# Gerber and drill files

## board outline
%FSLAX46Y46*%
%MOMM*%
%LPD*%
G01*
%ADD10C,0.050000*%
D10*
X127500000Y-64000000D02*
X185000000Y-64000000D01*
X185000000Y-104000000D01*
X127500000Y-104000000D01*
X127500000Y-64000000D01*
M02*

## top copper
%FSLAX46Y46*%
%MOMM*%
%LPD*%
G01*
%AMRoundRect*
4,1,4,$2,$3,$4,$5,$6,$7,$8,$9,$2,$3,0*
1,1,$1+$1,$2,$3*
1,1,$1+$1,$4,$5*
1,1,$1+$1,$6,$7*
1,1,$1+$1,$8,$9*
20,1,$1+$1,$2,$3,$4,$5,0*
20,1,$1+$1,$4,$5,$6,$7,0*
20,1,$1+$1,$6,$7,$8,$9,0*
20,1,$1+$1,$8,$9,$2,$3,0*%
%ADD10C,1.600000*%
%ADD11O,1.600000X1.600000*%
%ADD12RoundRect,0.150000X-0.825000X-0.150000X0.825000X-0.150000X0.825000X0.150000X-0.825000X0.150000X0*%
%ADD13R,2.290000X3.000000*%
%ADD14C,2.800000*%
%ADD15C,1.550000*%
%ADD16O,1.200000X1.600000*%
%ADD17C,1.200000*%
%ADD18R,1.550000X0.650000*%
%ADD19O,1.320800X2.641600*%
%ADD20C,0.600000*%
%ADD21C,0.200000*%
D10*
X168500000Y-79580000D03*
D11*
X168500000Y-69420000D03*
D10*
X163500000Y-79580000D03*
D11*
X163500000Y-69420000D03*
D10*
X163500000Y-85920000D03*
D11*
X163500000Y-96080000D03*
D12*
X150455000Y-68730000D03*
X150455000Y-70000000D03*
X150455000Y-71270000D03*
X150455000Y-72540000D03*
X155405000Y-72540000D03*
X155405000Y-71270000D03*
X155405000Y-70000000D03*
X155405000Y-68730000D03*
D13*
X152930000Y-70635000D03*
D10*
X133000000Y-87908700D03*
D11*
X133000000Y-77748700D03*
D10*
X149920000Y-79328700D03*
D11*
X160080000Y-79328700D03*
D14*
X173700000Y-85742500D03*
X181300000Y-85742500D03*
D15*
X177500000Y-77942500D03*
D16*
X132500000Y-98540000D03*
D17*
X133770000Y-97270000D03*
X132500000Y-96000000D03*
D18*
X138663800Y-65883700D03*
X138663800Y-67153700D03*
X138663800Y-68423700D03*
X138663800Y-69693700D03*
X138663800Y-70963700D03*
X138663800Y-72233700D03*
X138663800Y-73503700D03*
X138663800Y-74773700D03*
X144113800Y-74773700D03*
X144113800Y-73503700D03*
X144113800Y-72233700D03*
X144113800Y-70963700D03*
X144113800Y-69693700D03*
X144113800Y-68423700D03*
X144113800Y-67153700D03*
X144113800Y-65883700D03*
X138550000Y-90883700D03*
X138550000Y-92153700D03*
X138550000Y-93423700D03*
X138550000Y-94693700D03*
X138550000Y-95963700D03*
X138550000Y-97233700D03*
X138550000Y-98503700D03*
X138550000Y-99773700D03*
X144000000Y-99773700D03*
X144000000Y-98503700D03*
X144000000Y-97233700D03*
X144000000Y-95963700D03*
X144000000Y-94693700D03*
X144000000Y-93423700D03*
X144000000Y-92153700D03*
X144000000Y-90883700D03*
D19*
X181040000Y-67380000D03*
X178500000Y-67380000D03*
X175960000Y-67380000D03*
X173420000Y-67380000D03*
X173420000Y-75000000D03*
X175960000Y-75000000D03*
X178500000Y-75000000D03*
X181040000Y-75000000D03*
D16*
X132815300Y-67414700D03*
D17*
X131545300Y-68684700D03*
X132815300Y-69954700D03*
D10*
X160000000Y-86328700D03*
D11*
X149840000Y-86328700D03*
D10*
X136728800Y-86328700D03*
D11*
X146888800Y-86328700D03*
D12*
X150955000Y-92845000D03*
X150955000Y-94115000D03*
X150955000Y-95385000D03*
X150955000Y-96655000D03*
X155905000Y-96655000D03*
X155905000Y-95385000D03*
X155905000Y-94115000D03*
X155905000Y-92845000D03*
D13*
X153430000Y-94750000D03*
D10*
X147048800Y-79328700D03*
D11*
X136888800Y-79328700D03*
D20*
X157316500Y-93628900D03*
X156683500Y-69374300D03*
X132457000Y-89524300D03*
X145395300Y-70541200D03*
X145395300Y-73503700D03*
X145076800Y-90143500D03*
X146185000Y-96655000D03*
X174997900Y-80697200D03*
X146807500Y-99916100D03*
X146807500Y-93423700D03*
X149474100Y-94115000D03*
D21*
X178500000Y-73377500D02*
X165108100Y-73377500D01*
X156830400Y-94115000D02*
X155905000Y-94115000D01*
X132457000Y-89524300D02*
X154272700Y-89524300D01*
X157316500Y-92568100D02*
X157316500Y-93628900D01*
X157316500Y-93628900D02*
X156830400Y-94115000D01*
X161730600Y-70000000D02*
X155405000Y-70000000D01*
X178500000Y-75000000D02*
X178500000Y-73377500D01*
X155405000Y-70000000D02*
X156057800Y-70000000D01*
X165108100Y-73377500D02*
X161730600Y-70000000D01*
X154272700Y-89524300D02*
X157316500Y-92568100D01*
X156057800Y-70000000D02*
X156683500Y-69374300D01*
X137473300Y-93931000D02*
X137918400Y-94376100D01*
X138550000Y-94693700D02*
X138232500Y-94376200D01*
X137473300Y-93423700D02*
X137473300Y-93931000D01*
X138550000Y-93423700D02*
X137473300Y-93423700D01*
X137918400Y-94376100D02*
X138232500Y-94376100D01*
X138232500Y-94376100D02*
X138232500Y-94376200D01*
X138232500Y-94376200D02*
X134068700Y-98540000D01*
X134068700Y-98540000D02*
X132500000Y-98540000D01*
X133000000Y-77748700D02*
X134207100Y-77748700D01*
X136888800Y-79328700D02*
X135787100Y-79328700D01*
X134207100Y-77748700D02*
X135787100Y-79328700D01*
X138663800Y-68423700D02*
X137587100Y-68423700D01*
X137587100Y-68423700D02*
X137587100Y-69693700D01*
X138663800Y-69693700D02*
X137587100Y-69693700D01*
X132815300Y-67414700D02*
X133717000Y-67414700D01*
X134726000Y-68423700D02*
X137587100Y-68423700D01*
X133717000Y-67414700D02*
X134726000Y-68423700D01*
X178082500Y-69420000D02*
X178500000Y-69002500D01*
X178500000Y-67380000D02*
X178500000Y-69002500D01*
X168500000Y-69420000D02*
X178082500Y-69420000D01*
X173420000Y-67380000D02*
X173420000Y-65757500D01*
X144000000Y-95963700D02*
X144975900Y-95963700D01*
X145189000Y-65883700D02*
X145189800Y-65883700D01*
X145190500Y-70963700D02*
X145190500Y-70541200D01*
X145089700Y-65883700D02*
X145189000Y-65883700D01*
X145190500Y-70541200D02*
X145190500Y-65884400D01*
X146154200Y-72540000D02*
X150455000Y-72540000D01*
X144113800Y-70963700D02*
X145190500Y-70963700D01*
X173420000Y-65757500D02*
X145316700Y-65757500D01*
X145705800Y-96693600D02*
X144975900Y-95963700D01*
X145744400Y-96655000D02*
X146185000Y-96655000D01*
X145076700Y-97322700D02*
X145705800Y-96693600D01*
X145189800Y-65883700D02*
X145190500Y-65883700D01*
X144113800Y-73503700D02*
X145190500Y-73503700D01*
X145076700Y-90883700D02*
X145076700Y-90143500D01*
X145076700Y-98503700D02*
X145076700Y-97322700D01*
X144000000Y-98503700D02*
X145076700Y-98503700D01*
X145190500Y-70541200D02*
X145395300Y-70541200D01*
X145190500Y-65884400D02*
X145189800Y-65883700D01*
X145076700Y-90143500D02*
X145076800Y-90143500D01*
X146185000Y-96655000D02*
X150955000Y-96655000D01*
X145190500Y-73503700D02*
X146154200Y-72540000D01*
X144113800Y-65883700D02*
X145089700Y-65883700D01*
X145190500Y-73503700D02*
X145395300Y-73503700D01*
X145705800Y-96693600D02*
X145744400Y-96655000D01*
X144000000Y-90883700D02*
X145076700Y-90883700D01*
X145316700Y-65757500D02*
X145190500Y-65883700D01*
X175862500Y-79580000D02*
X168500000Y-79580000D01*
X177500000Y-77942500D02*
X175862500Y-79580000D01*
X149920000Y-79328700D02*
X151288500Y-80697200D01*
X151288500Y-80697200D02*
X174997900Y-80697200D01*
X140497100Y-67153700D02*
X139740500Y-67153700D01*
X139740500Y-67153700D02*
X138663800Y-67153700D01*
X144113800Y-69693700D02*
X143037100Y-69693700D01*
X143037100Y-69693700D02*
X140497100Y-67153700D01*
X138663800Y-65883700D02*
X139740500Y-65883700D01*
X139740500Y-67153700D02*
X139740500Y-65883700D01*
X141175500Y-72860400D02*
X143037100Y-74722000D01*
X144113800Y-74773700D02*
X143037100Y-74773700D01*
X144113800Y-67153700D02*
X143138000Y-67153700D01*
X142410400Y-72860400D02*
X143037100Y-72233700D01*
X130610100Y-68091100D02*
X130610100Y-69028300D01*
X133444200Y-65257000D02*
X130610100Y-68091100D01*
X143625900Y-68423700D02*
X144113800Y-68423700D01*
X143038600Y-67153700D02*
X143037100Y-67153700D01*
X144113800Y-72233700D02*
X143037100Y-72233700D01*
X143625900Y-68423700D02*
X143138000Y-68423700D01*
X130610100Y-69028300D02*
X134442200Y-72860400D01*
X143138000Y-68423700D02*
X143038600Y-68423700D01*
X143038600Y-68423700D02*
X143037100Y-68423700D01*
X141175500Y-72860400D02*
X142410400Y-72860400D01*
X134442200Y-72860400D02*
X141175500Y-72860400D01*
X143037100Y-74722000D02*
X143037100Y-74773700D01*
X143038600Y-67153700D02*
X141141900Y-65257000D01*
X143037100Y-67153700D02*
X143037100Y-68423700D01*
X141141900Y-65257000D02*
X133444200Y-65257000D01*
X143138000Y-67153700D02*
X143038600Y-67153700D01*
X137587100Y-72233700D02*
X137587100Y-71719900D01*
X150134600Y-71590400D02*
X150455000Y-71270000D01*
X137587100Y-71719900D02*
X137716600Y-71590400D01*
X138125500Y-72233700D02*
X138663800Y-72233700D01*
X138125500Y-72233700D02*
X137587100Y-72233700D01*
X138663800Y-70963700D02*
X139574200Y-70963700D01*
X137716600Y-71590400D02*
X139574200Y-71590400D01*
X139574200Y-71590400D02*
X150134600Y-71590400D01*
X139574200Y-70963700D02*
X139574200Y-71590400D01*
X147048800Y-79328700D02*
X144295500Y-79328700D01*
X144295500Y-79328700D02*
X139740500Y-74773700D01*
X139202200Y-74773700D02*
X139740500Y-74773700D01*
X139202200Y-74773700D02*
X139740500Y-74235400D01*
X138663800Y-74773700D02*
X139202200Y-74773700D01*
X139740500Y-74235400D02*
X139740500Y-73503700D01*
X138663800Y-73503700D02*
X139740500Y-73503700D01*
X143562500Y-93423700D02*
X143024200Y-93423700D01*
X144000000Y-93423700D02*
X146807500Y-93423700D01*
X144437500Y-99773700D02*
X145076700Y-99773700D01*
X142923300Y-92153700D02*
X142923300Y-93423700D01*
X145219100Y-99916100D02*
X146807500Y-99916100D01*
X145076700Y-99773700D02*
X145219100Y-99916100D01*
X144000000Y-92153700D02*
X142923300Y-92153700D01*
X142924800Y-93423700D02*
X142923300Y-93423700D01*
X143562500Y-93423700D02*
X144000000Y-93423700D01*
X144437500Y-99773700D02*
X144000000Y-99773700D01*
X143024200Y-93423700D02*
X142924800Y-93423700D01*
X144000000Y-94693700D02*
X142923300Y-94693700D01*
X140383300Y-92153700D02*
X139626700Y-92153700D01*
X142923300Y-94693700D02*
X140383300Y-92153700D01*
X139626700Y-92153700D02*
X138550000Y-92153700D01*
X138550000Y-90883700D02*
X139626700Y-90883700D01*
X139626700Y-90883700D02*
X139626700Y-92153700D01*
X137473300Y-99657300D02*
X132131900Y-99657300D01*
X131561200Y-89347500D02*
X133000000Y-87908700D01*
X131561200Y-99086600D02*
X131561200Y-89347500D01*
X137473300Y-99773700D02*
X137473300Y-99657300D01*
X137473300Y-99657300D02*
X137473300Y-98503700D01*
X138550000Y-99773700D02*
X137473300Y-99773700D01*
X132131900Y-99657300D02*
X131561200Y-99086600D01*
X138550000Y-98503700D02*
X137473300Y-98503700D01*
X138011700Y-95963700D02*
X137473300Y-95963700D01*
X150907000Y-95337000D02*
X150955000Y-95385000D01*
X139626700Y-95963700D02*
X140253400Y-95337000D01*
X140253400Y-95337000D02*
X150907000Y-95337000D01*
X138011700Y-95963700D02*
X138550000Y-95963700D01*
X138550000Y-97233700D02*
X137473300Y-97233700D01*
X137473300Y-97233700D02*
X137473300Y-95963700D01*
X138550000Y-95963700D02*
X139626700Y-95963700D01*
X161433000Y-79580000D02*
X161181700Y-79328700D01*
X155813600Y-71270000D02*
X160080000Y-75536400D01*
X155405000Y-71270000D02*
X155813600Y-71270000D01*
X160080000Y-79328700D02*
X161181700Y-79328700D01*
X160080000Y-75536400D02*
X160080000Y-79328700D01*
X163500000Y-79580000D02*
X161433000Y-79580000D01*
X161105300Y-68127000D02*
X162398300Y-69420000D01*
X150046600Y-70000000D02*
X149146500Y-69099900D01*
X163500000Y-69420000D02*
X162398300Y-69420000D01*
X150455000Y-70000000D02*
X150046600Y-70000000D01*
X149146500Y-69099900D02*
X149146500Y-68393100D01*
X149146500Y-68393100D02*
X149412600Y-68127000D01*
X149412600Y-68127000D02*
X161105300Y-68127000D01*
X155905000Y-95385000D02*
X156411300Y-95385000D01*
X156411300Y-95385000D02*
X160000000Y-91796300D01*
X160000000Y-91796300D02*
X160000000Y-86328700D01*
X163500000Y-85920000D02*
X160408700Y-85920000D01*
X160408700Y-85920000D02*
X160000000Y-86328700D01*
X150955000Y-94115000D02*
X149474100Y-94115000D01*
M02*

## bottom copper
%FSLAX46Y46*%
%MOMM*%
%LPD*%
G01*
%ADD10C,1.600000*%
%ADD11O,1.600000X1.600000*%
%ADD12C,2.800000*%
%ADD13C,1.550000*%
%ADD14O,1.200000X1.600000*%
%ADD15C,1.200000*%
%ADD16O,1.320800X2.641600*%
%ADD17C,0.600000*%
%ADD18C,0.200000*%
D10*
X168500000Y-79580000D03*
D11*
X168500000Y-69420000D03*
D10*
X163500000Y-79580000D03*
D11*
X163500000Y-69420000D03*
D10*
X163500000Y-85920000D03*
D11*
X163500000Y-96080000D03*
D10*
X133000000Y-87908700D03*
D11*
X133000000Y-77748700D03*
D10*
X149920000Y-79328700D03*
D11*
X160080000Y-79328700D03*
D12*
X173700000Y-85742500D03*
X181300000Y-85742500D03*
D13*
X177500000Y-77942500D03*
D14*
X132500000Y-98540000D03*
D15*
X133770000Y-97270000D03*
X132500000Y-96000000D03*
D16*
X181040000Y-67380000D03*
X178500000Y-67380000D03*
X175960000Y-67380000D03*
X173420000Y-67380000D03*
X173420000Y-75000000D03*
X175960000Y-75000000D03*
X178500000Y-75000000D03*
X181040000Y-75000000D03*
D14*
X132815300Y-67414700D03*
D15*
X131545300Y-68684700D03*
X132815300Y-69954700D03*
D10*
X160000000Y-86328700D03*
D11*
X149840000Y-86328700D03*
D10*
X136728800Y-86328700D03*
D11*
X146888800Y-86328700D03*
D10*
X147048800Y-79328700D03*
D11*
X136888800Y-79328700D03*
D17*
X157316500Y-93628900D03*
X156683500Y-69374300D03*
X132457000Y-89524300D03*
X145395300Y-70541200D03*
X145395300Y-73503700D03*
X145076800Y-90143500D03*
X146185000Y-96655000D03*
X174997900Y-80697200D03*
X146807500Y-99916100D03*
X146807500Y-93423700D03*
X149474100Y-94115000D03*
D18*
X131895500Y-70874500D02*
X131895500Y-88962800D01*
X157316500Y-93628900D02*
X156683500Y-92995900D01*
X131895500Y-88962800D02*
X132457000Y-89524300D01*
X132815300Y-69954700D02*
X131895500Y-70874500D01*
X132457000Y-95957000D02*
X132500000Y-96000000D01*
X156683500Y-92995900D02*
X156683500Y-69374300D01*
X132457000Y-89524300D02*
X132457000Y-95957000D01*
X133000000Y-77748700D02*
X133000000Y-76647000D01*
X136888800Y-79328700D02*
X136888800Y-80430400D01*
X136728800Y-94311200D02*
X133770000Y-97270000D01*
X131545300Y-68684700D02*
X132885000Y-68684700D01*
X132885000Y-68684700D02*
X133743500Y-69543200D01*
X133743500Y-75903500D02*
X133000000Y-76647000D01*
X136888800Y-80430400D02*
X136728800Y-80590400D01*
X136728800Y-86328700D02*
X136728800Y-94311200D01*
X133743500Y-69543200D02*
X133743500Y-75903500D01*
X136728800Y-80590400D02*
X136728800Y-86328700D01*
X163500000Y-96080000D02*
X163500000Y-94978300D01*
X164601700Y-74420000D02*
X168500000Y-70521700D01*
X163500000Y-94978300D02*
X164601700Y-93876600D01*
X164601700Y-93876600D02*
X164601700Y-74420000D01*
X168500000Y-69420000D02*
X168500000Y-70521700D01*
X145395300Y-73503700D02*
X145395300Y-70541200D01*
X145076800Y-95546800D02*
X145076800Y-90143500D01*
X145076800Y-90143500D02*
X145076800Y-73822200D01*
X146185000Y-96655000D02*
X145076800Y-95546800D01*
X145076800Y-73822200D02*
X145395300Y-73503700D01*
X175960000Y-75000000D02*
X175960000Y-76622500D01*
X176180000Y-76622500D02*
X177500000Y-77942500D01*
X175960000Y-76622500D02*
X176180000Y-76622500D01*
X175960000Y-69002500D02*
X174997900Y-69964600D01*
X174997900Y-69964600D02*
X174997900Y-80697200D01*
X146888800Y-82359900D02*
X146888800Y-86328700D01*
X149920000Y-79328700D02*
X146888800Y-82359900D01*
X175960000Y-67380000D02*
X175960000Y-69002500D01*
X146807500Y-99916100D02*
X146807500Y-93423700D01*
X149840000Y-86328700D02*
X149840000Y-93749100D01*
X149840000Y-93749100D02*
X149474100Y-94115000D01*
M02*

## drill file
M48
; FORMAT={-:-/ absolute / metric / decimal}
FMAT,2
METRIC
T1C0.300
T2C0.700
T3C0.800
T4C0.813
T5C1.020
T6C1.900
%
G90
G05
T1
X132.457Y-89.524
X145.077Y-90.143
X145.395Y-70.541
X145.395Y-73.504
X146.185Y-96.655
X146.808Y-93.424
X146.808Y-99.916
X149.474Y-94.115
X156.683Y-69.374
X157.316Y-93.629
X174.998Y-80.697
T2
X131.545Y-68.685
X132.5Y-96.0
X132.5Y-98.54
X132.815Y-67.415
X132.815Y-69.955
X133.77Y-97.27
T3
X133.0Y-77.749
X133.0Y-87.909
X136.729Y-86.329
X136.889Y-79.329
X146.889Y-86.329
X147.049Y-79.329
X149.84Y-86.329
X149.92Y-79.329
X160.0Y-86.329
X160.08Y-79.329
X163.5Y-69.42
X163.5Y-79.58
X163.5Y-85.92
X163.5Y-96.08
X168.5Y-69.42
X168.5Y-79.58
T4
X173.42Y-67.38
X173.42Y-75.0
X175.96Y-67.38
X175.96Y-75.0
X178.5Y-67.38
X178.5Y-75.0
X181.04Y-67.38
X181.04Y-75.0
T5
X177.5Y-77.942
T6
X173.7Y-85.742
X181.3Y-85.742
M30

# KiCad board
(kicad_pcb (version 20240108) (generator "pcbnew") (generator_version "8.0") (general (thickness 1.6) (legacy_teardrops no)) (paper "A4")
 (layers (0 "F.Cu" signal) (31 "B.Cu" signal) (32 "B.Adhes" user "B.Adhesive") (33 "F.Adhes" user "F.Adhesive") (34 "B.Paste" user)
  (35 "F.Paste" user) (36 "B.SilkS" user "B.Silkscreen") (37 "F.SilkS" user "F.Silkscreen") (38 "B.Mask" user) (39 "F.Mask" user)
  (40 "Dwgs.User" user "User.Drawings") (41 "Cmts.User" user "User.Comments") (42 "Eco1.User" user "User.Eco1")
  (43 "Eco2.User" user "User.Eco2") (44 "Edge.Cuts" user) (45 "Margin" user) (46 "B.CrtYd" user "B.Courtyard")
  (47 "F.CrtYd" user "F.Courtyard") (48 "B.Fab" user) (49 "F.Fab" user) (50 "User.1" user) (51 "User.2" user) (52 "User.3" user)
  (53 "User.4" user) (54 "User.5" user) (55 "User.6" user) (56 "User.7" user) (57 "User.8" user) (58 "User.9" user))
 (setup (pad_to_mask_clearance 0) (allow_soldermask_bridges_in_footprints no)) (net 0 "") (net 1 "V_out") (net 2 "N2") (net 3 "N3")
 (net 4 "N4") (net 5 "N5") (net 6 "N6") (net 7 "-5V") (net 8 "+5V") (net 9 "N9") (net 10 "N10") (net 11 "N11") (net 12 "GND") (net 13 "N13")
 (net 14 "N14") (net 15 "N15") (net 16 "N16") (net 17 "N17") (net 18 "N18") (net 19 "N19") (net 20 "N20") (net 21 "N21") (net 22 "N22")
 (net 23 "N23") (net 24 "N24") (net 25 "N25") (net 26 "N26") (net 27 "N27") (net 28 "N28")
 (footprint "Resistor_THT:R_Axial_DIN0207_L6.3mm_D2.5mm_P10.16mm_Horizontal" (layer "F.Cu") (at 168.5 79.58 90)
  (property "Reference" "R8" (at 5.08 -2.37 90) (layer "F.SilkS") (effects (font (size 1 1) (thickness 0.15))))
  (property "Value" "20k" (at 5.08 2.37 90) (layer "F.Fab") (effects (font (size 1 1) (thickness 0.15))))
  (pad "1" thru_hole circle (at 0 0 90) (size 1.6 1.6) (drill 0.8) (layers "*.Cu" "*.Mask") (remove_unused_layers no) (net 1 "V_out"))
  (pad "2" thru_hole oval (at 10.16 0 90) (size 1.6 1.6) (drill 0.8) (layers "*.Cu" "*.Mask") (remove_unused_layers no) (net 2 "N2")))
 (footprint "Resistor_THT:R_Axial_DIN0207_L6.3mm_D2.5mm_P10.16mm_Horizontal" (layer "F.Cu") (at 163.5 79.58 90)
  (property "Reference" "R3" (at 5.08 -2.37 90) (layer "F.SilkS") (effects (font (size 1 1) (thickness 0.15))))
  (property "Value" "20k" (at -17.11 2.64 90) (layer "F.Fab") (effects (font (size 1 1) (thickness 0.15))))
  (pad "1" thru_hole circle (at 0 0 90) (size 1.6 1.6) (drill 0.8) (layers "*.Cu" "*.Mask") (remove_unused_layers no) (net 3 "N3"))
  (pad "2" thru_hole oval (at 10.16 0 90) (size 1.6 1.6) (drill 0.8) (layers "*.Cu" "*.Mask") (remove_unused_layers no) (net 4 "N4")))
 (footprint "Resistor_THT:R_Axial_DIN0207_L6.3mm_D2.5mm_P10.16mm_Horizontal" (layer "F.Cu") (at 163.5 85.92 -90)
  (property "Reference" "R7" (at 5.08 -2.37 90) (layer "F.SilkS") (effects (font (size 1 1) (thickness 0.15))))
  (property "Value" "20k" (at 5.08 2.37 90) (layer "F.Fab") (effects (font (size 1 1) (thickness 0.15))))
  (pad "1" thru_hole circle (at 0 0 270) (size 1.6 1.6) (drill 0.8) (layers "*.Cu" "*.Mask") (remove_unused_layers no) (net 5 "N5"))
  (pad "2" thru_hole oval (at 10.16 0 270) (size 1.6 1.6) (drill 0.8) (layers "*.Cu" "*.Mask") (remove_unused_layers no) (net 2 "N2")))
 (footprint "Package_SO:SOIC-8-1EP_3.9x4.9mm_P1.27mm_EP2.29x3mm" (layer "F.Cu") (at 152.93 70.635)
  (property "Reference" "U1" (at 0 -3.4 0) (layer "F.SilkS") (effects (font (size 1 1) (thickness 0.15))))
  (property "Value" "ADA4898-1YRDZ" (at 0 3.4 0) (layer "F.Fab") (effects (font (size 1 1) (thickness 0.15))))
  (pad "" smd roundrect (at -0.57 -0.75) (size 0.92 1.21) (layers "F.Paste") (roundrect_rratio 0.25))
  (pad "" smd roundrect (at -0.57 0.75) (size 0.92 1.21) (layers "F.Paste") (roundrect_rratio 0.25))
  (pad "" smd roundrect (at 0.57 -0.75) (size 0.92 1.21) (layers "F.Paste") (roundrect_rratio 0.25))
  (pad "" smd roundrect (at 0.57 0.75) (size 0.92 1.21) (layers "F.Paste") (roundrect_rratio 0.25))
  (pad "1" smd roundrect (at -2.475 -1.905) (size 1.95 0.6) (layers "F.Cu" "F.Paste" "F.Mask") (roundrect_rratio 0.25))
  (pad "2" smd roundrect (at -2.475 -0.635) (size 1.95 0.6) (layers "F.Cu" "F.Paste" "F.Mask") (roundrect_rratio 0.25) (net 4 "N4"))
  (pad "3" smd roundrect (at -2.475 0.635) (size 1.95 0.6) (layers "F.Cu" "F.Paste" "F.Mask") (roundrect_rratio 0.25) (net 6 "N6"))
  (pad "4" smd roundrect (at -2.475 1.905) (size 1.95 0.6) (layers "F.Cu" "F.Paste" "F.Mask") (roundrect_rratio 0.25) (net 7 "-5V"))
  (pad "5" smd roundrect (at 2.475 1.905) (size 1.95 0.6) (layers "F.Cu" "F.Paste" "F.Mask") (roundrect_rratio 0.25))
  (pad "6" smd roundrect (at 2.475 0.635) (size 1.95 0.6) (layers "F.Cu" "F.Paste" "F.Mask") (roundrect_rratio 0.25) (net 3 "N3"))
  (pad "7" smd roundrect (at 2.475 -0.635) (size 1.95 0.6) (layers "F.Cu" "F.Paste" "F.Mask") (roundrect_rratio 0.25) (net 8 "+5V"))
  (pad "8" smd roundrect (at 2.475 -1.905) (size 1.95 0.6) (layers "F.Cu" "F.Paste" "F.Mask") (roundrect_rratio 0.25) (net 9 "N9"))
  (pad "9" smd rect (at 0 0) (size 2.29 3) (layers "F.Cu" "F.Mask") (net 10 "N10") (zone_connect 2)))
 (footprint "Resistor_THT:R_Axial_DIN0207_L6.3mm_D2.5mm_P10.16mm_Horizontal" (layer "F.Cu") (at 133 87.9087 90)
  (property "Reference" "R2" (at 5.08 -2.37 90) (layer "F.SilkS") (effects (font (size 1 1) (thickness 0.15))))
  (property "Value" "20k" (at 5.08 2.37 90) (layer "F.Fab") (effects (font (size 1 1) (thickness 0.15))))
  (pad "1" thru_hole circle (at 0 0 90) (size 1.6 1.6) (drill 0.8) (layers "*.Cu" "*.Mask") (remove_unused_layers no) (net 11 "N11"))
  (pad "2" thru_hole oval (at 10.16 0 90) (size 1.6 1.6) (drill 0.8) (layers "*.Cu" "*.Mask") (remove_unused_layers no) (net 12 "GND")))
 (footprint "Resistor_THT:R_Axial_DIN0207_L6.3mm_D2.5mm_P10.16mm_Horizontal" (layer "F.Cu") (at 149.92 79.3287)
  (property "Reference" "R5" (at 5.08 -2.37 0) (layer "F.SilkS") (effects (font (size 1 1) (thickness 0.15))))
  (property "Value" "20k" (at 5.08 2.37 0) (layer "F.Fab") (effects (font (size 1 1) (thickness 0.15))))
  (pad "1" thru_hole circle (at 0 0) (size 1.6 1.6) (drill 0.8) (layers "*.Cu" "*.Mask") (remove_unused_layers no) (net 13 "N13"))
  (pad "2" thru_hole oval (at 10.16 0) (size 1.6 1.6) (drill 0.8) (layers "*.Cu" "*.Mask") (remove_unused_layers no) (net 3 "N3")))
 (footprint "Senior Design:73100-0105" (layer "F.Cu") (at 177.5 103.3425)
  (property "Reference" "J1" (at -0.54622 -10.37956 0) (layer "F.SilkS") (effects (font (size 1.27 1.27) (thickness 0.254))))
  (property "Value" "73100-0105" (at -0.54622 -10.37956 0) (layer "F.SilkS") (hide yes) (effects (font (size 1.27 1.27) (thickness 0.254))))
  (pad "1" thru_hole circle (at -3.8 -17.6) (size 2.8 2.8) (drill 1.9) (layers "*.Cu" "*.Mask") (remove_unused_layers no) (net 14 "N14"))
  (pad "2" thru_hole circle (at 3.8 -17.6) (size 2.8 2.8) (drill 1.9) (layers "*.Cu" "*.Mask") (remove_unused_layers no) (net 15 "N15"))
  (pad "3" thru_hole circle (at 0 -25.4) (size 1.55 1.55) (drill 1.02) (layers "*.Cu" "*.Mask") (remove_unused_layers no) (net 1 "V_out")))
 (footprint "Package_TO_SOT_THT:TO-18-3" (layer "F.Cu") (at 132.5 98.54 90)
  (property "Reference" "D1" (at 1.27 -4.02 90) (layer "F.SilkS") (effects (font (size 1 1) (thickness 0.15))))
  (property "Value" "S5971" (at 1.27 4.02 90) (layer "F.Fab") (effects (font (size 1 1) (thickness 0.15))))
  (pad "1" thru_hole oval (at 0 0 90) (size 1.6 1.2) (drill 0.7) (layers "*.Cu" "*.Mask") (remove_unused_layers no) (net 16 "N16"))
  (pad "2" thru_hole circle (at 1.27 1.27 90) (size 1.2 1.2) (drill 0.7) (layers "*.Cu" "*.Mask") (remove_unused_layers no) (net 12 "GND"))
  (pad "3" thru_hole circle (at 2.54 0 90) (size 1.2 1.2) (drill 0.7) (layers "*.Cu" "*.Mask") (remove_unused_layers no) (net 8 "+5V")))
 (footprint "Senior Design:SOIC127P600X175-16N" (layer "F.Cu") (at 141.3888 70.3287)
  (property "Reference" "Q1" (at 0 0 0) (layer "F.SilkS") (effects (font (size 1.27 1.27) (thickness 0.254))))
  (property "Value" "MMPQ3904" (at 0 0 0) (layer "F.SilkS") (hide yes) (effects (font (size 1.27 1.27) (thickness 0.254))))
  (pad "1" smd rect (at -2.725 -4.445 90) (size 0.65 1.55) (layers "F.Cu" "F.Paste" "F.Mask") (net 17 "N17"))
  (pad "2" smd rect (at -2.725 -3.175 90) (size 0.65 1.55) (layers "F.Cu" "F.Paste" "F.Mask") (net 17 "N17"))
  (pad "3" smd rect (at -2.725 -1.905 90) (size 0.65 1.55) (layers "F.Cu" "F.Paste" "F.Mask") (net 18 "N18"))
  (pad "4" smd rect (at -2.725 -0.635 90) (size 0.65 1.55) (layers "F.Cu" "F.Paste" "F.Mask") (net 18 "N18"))
  (pad "5" smd rect (at -2.725 0.635 90) (size 0.65 1.55) (layers "F.Cu" "F.Paste" "F.Mask") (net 6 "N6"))
  (pad "6" smd rect (at -2.725 1.905 90) (size 0.65 1.55) (layers "F.Cu" "F.Paste" "F.Mask") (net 6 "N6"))
  (pad "7" smd rect (at -2.725 3.175 90) (size 0.65 1.55) (layers "F.Cu" "F.Paste" "F.Mask") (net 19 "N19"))
  (pad "8" smd rect (at -2.725 4.445 90) (size 0.65 1.55) (layers "F.Cu" "F.Paste" "F.Mask") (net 19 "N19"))
  (pad "9" smd rect (at 2.725 4.445 90) (size 0.65 1.55) (layers "F.Cu" "F.Paste" "F.Mask") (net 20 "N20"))
  (pad "10" smd rect (at 2.725 3.175 90) (size 0.65 1.55) (layers "F.Cu" "F.Paste" "F.Mask") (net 7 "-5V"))
  (pad "11" smd rect (at 2.725 1.905 90) (size 0.65 1.55) (layers "F.Cu" "F.Paste" "F.Mask") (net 20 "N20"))
  (pad "12" smd rect (at 2.725 0.635 90) (size 0.65 1.55) (layers "F.Cu" "F.Paste" "F.Mask") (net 7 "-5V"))
  (pad "13" smd rect (at 2.725 -0.635 90) (size 0.65 1.55) (layers "F.Cu" "F.Paste" "F.Mask") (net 17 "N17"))
  (pad "14" smd rect (at 2.725 -1.905 90) (size 0.65 1.55) (layers "F.Cu" "F.Paste" "F.Mask") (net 20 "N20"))
  (pad "15" smd rect (at 2.725 -3.175 90) (size 0.65 1.55) (layers "F.Cu" "F.Paste" "F.Mask") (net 20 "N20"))
  (pad "16" smd rect (at 2.725 -4.445 90) (size 0.65 1.55) (layers "F.Cu" "F.Paste" "F.Mask") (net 7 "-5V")))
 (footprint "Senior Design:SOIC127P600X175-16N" (layer "F.Cu") (at 141.275 95.3287)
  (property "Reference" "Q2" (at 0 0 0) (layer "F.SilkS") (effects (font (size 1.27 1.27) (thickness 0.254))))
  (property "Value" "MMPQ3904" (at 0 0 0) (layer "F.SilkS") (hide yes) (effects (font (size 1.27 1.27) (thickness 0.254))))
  (pad "1" smd rect (at -2.725 -4.445 90) (size 0.65 1.55) (layers "F.Cu" "F.Paste" "F.Mask") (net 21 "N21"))
  (pad "2" smd rect (at -2.725 -3.175 90) (size 0.65 1.55) (layers "F.Cu" "F.Paste" "F.Mask") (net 21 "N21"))
  (pad "3" smd rect (at -2.725 -1.905 90) (size 0.65 1.55) (layers "F.Cu" "F.Paste" "F.Mask") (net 16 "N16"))
  (pad "4" smd rect (at -2.725 -0.635 90) (size 0.65 1.55) (layers "F.Cu" "F.Paste" "F.Mask") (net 16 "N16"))
  (pad "5" smd rect (at -2.725 0.635 90) (size 0.65 1.55) (layers "F.Cu" "F.Paste" "F.Mask") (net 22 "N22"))
  (pad "6" smd rect (at -2.725 1.905 90) (size 0.65 1.55) (layers "F.Cu" "F.Paste" "F.Mask") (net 22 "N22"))
  (pad "7" smd rect (at -2.725 3.175 90) (size 0.65 1.55) (layers "F.Cu" "F.Paste" "F.Mask") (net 11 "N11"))
  (pad "8" smd rect (at -2.725 4.445 90) (size 0.65 1.55) (layers "F.Cu" "F.Paste" "F.Mask") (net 11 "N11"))
  (pad "9" smd rect (at 2.725 4.445 90) (size 0.65 1.55) (layers "F.Cu" "F.Paste" "F.Mask") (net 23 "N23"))
  (pad "10" smd rect (at 2.725 3.175 90) (size 0.65 1.55) (layers "F.Cu" "F.Paste" "F.Mask") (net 7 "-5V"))
  (pad "11" smd rect (at 2.725 1.905 90) (size 0.65 1.55) (layers "F.Cu" "F.Paste" "F.Mask") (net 23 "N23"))
  (pad "12" smd rect (at 2.725 0.635 90) (size 0.65 1.55) (layers "F.Cu" "F.Paste" "F.Mask") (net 7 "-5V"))
  (pad "13" smd rect (at 2.725 -0.635 90) (size 0.65 1.55) (layers "F.Cu" "F.Paste" "F.Mask") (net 21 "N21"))
  (pad "14" smd rect (at 2.725 -1.905 90) (size 0.65 1.55) (layers "F.Cu" "F.Paste" "F.Mask") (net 23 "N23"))
  (pad "15" smd rect (at 2.725 -3.175 90) (size 0.65 1.55) (layers "F.Cu" "F.Paste" "F.Mask") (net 23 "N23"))
  (pad "16" smd rect (at 2.725 -4.445 90) (size 0.65 1.55) (layers "F.Cu" "F.Paste" "F.Mask") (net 7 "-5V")))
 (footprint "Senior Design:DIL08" (layer "F.Cu") (at 177.23 71.19 180)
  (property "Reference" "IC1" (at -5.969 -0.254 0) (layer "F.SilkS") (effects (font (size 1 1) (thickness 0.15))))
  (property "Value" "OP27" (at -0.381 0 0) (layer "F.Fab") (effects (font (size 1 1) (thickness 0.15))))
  (pad "1" thru_hole oval (at -3.81 3.81 180) (size 1.3208 2.6416) (drill 0.8128) (layers "*.Cu" "*.Mask") (remove_unused_layers no)
   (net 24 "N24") (solder_mask_margin 0.102))
  (pad "2" thru_hole oval (at -1.27 3.81 180) (size 1.3208 2.6416) (drill 0.8128) (layers "*.Cu" "*.Mask") (remove_unused_layers no)
   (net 2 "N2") (solder_mask_margin 0.102))
  (pad "3" thru_hole oval (at 1.27 3.81 180) (size 1.3208 2.6416) (drill 0.8128) (layers "*.Cu" "*.Mask") (remove_unused_layers no)
   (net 13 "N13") (solder_mask_margin 0.102))
  (pad "4" thru_hole oval (at 3.81 3.81 180) (size 1.3208 2.6416) (drill 0.8128) (layers "*.Cu" "*.Mask") (remove_unused_layers no)
   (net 7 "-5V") (solder_mask_margin 0.102))
  (pad "5" thru_hole oval (at 3.81 -3.81 180) (size 1.3208 2.6416) (drill 0.8128) (layers "*.Cu" "*.Mask") (remove_unused_layers no)
   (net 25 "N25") (solder_mask_margin 0.102))
  (pad "6" thru_hole oval (at 1.27 -3.81 180) (size 1.3208 2.6416) (drill 0.8128) (layers "*.Cu" "*.Mask") (remove_unused_layers no)
   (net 1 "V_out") (solder_mask_margin 0.102))
  (pad "7" thru_hole oval (at -1.27 -3.81 180) (size 1.3208 2.6416) (drill 0.8128) (layers "*.Cu" "*.Mask") (remove_unused_layers no)
   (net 8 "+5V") (solder_mask_margin 0.102))
  (pad "8" thru_hole oval (at -3.81 -3.81 180) (size 1.3208 2.6416) (drill 0.8128) (layers "*.Cu" "*.Mask") (remove_unused_layers no)
   (solder_mask_margin 0.102)))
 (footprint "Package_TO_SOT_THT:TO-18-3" (layer "F.Cu") (at 132.8153 67.4147 -90)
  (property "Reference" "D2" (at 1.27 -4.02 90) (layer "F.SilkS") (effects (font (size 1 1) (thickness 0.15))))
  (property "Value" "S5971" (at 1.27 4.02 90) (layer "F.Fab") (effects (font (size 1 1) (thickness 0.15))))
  (pad "1" thru_hole oval (at 0 0 270) (size 1.6 1.2) (drill 0.7) (layers "*.Cu" "*.Mask") (remove_unused_layers no) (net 18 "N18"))
  (pad "2" thru_hole circle (at 1.27 1.27 270) (size 1.2 1.2) (drill 0.7) (layers "*.Cu" "*.Mask") (remove_unused_layers no) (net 12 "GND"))
  (pad "3" thru_hole circle (at 2.54 0 270) (size 1.2 1.2) (drill 0.7) (layers "*.Cu" "*.Mask") (remove_unused_layers no) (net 8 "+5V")))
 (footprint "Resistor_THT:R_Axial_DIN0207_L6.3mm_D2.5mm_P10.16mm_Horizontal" (layer "F.Cu") (at 160 86.3287 180)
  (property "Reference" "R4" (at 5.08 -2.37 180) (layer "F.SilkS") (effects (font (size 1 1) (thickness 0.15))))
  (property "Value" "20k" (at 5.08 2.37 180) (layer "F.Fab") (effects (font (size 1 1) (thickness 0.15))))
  (pad "1" thru_hole circle (at 0 0 180) (size 1.6 1.6) (drill 0.8) (layers "*.Cu" "*.Mask") (remove_unused_layers no) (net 5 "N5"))
  (pad "2" thru_hole oval (at 10.16 0 180) (size 1.6 1.6) (drill 0.8) (layers "*.Cu" "*.Mask") (remove_unused_layers no) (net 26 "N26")))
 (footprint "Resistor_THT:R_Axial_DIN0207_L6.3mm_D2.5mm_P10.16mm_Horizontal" (layer "F.Cu") (at 136.7288 86.3287)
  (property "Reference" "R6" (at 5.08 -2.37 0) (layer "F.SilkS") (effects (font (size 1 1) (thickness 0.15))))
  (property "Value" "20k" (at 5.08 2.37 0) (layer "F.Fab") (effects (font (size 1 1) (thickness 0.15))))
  (pad "1" thru_hole circle (at 0 0) (size 1.6 1.6) (drill 0.8) (layers "*.Cu" "*.Mask") (remove_unused_layers no) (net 12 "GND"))
  (pad "2" thru_hole oval (at 10.16 0) (size 1.6 1.6) (drill 0.8) (layers "*.Cu" "*.Mask") (remove_unused_layers no) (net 13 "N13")))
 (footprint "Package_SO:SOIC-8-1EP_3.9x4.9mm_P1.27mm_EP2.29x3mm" (layer "F.Cu") (at 153.43 94.75)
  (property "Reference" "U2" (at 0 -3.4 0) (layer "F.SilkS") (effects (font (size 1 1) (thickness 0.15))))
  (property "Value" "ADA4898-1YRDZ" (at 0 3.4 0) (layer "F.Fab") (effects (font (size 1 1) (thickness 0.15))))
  (pad "" smd roundrect (at -0.57 -0.75) (size 0.92 1.21) (layers "F.Paste") (roundrect_rratio 0.25))
  (pad "" smd roundrect (at -0.57 0.75) (size 0.92 1.21) (layers "F.Paste") (roundrect_rratio 0.25))
  (pad "" smd roundrect (at 0.57 -0.75) (size 0.92 1.21) (layers "F.Paste") (roundrect_rratio 0.25))
  (pad "" smd roundrect (at 0.57 0.75) (size 0.92 1.21) (layers "F.Paste") (roundrect_rratio 0.25))
  (pad "1" smd roundrect (at -2.475 -1.905) (size 1.95 0.6) (layers "F.Cu" "F.Paste" "F.Mask") (roundrect_rratio 0.25))
  (pad "2" smd roundrect (at -2.475 -0.635) (size 1.95 0.6) (layers "F.Cu" "F.Paste" "F.Mask") (roundrect_rratio 0.25) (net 26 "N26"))
  (pad "3" smd roundrect (at -2.475 0.635) (size 1.95 0.6) (layers "F.Cu" "F.Paste" "F.Mask") (roundrect_rratio 0.25) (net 22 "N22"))
  (pad "4" smd roundrect (at -2.475 1.905) (size 1.95 0.6) (layers "F.Cu" "F.Paste" "F.Mask") (roundrect_rratio 0.25) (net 7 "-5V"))
  (pad "5" smd roundrect (at 2.475 1.905) (size 1.95 0.6) (layers "F.Cu" "F.Paste" "F.Mask") (roundrect_rratio 0.25))
  (pad "6" smd roundrect (at 2.475 0.635) (size 1.95 0.6) (layers "F.Cu" "F.Paste" "F.Mask") (roundrect_rratio 0.25) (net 5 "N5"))
  (pad "7" smd roundrect (at 2.475 -0.635) (size 1.95 0.6) (layers "F.Cu" "F.Paste" "F.Mask") (roundrect_rratio 0.25) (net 8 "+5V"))
  (pad "8" smd roundrect (at 2.475 -1.905) (size 1.95 0.6) (layers "F.Cu" "F.Paste" "F.Mask") (roundrect_rratio 0.25) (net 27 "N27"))
  (pad "9" smd rect (at 0 0) (size 2.29 3) (layers "F.Cu" "F.Mask") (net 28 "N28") (zone_connect 2)))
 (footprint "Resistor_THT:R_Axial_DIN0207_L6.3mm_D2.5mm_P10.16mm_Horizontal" (layer "F.Cu") (at 147.0488 79.3287 180)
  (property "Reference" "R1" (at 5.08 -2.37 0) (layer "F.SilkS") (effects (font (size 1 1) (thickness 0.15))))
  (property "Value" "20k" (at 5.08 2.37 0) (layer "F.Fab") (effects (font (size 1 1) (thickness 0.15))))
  (pad "1" thru_hole circle (at 0 0 180) (size 1.6 1.6) (drill 0.8) (layers "*.Cu" "*.Mask") (remove_unused_layers no) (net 19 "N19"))
  (pad "2" thru_hole oval (at 10.16 0 180) (size 1.6 1.6) (drill 0.8) (layers "*.Cu" "*.Mask") (remove_unused_layers no) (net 12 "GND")))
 (gr_rect (start 127.5 64) (end 185 104) (stroke (width 0.05) (type default)) (fill none) (layer "Edge.Cuts"))
 (segment (start 178.5 73.3775) (end 165.1081 73.3775) (width 0.2) (layer "F.Cu") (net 8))
 (segment (start 156.8304 94.115) (end 155.905 94.115) (width 0.2) (layer "F.Cu") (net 8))
 (segment (start 132.457 89.5243) (end 154.2727 89.5243) (width 0.2) (layer "F.Cu") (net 8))
 (segment (start 157.3165 92.5681) (end 157.3165 93.6289) (width 0.2) (layer "F.Cu") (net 8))
 (segment (start 157.3165 93.6289) (end 156.8304 94.115) (width 0.2) (layer "F.Cu") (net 8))
 (segment (start 161.7306 70) (end 155.405 70) (width 0.2) (layer "F.Cu") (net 8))
 (segment (start 178.5 75) (end 178.5 73.3775) (width 0.2) (layer "F.Cu") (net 8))
 (segment (start 155.405 70) (end 156.0578 70) (width 0.2) (layer "F.Cu") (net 8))
 (segment (start 165.1081 73.3775) (end 161.7306 70) (width 0.2) (layer "F.Cu") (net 8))
 (segment (start 154.2727 89.5243) (end 157.3165 92.5681) (width 0.2) (layer "F.Cu") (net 8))
 (segment (start 156.0578 70) (end 156.6835 69.3743) (width 0.2) (layer "F.Cu") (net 8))
 (via (at 157.3165 93.6289) (size 0.6) (drill 0.3) (layers "F.Cu" "B.Cu") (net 8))
 (via (at 156.6835 69.3743) (size 0.6) (drill 0.3) (layers "F.Cu" "B.Cu") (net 8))
 (via (at 132.457 89.5243) (size 0.6) (drill 0.3) (layers "F.Cu" "B.Cu") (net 8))
 (segment (start 131.8955 70.8745) (end 131.8955 88.9628) (width 0.2) (layer "B.Cu") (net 8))
 (segment (start 157.3165 93.6289) (end 156.6835 92.9959) (width 0.2) (layer "B.Cu") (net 8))
 (segment (start 131.8955 88.9628) (end 132.457 89.5243) (width 0.2) (layer "B.Cu") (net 8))
 (segment (start 132.8153 69.9547) (end 131.8955 70.8745) (width 0.2) (layer "B.Cu") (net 8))
 (segment (start 132.457 95.957) (end 132.5 96) (width 0.2) (layer "B.Cu") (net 8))
 (segment (start 156.6835 92.9959) (end 156.6835 69.3743) (width 0.2) (layer "B.Cu") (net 8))
 (segment (start 132.457 89.5243) (end 132.457 95.957) (width 0.2) (layer "B.Cu") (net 8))
 (segment (start 137.4733 93.931) (end 137.9184 94.3761) (width 0.2) (layer "F.Cu") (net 16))
 (segment (start 138.55 94.6937) (end 138.2325 94.3762) (width 0.2) (layer "F.Cu") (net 16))
 (segment (start 137.4733 93.4237) (end 137.4733 93.931) (width 0.2) (layer "F.Cu") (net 16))
 (segment (start 138.55 93.4237) (end 137.4733 93.4237) (width 0.2) (layer "F.Cu") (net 16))
 (segment (start 137.9184 94.3761) (end 138.2325 94.3761) (width 0.2) (layer "F.Cu") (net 16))
 (segment (start 138.2325 94.3761) (end 138.2325 94.3762) (width 0.2) (layer "F.Cu") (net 16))
 (segment (start 138.2325 94.3762) (end 134.0687 98.54) (width 0.2) (layer "F.Cu") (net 16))
 (segment (start 134.0687 98.54) (end 132.5 98.54) (width 0.2) (layer "F.Cu") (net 16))
 (segment (start 133 77.7487) (end 134.2071 77.7487) (width 0.2) (layer "F.Cu") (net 12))
 (segment (start 136.8888 79.3287) (end 135.7871 79.3287) (width 0.2) (layer "F.Cu") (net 12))
 (segment (start 134.2071 77.7487) (end 135.7871 79.3287) (width 0.2) (layer "F.Cu") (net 12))
 (segment (start 133 77.7487) (end 133 76.647) (width 0.2) (layer "B.Cu") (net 12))
 (segment (start 136.8888 79.3287) (end 136.8888 80.4304) (width 0.2) (layer "B.Cu") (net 12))
 (segment (start 136.7288 94.3112) (end 133.77 97.27) (width 0.2) (layer "B.Cu") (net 12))
 (segment (start 131.5453 68.6847) (end 132.885 68.6847) (width 0.2) (layer "B.Cu") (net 12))
 (segment (start 132.885 68.6847) (end 133.7435 69.5432) (width 0.2) (layer "B.Cu") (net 12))
 (segment (start 133.7435 75.9035) (end 133 76.647) (width 0.2) (layer "B.Cu") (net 12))
 (segment (start 136.8888 80.4304) (end 136.7288 80.5904) (width 0.2) (layer "B.Cu") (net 12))
 (segment (start 136.7288 86.3287) (end 136.7288 94.3112) (width 0.2) (layer "B.Cu") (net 12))
 (segment (start 133.7435 69.5432) (end 133.7435 75.9035) (width 0.2) (layer "B.Cu") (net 12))
 (segment (start 136.7288 80.5904) (end 136.7288 86.3287) (width 0.2) (layer "B.Cu") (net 12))
 (segment (start 138.6638 68.4237) (end 137.5871 68.4237) (width 0.2) (layer "F.Cu") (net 18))
 (segment (start 137.5871 68.4237) (end 137.5871 69.6937) (width 0.2) (layer "F.Cu") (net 18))
 (segment (start 138.6638 69.6937) (end 137.5871 69.6937) (width 0.2) (layer "F.Cu") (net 18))
 (segment (start 132.8153 67.4147) (end 133.717 67.4147) (width 0.2) (layer "F.Cu") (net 18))
 (segment (start 134.726 68.4237) (end 137.5871 68.4237) (width 0.2) (layer "F.Cu") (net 18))
 (segment (start 133.717 67.4147) (end 134.726 68.4237) (width 0.2) (layer "F.Cu") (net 18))
 (segment (start 178.0825 69.42) (end 178.5 69.0025) (width 0.2) (layer "F.Cu") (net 2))
 (segment (start 178.5 67.38) (end 178.5 69.0025) (width 0.2) (layer "F.Cu") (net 2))
 (segment (start 168.5 69.42) (end 178.0825 69.42) (width 0.2) (layer "F.Cu") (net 2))
 (segment (start 163.5 96.08) (end 163.5 94.9783) (width 0.2) (layer "B.Cu") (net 2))
 (segment (start 164.6017 74.42) (end 168.5 70.5217) (width 0.2) (layer "B.Cu") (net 2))
 (segment (start 163.5 94.9783) (end 164.6017 93.8766) (width 0.2) (layer "B.Cu") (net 2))
 (segment (start 164.6017 93.8766) (end 164.6017 74.42) (width 0.2) (layer "B.Cu") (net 2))
 (segment (start 168.5 69.42) (end 168.5 70.5217) (width 0.2) (layer "B.Cu") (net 2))
 (segment (start 173.42 67.38) (end 173.42 65.7575) (width 0.2) (layer "F.Cu") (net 7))
 (segment (start 144 95.9637) (end 144.9759 95.9637) (width 0.2) (layer "F.Cu") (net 7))
 (segment (start 145.189 65.8837) (end 145.1898 65.8837) (width 0.2) (layer "F.Cu") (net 7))
 (segment (start 145.1905 70.9637) (end 145.1905 70.5412) (width 0.2) (layer "F.Cu") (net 7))
 (segment (start 145.0897 65.8837) (end 145.189 65.8837) (width 0.2) (layer "F.Cu") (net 7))
 (segment (start 145.1905 70.5412) (end 145.1905 65.8844) (width 0.2) (layer "F.Cu") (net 7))
 (segment (start 146.1542 72.54) (end 150.455 72.54) (width 0.2) (layer "F.Cu") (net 7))
 (segment (start 144.1138 70.9637) (end 145.1905 70.9637) (width 0.2) (layer "F.Cu") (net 7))
 (segment (start 173.42 65.7575) (end 145.3167 65.7575) (width 0.2) (layer "F.Cu") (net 7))
 (segment (start 145.7058 96.6936) (end 144.9759 95.9637) (width 0.2) (layer "F.Cu") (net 7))
 (segment (start 145.7444 96.655) (end 146.185 96.655) (width 0.2) (layer "F.Cu") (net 7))
 (segment (start 145.0767 97.3227) (end 145.7058 96.6936) (width 0.2) (layer "F.Cu") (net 7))
 (segment (start 145.1898 65.8837) (end 145.1905 65.8837) (width 0.2) (layer "F.Cu") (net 7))
 (segment (start 144.1138 73.5037) (end 145.1905 73.5037) (width 0.2) (layer "F.Cu") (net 7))
 (segment (start 145.0767 90.8837) (end 145.0767 90.1435) (width 0.2) (layer "F.Cu") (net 7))
 (segment (start 145.0767 98.5037) (end 145.0767 97.3227) (width 0.2) (layer "F.Cu") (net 7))
 (segment (start 144 98.5037) (end 145.0767 98.5037) (width 0.2) (layer "F.Cu") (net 7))
 (segment (start 145.1905 70.5412) (end 145.3953 70.5412) (width 0.2) (layer "F.Cu") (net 7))
 (segment (start 145.1905 65.8844) (end 145.1898 65.8837) (width 0.2) (layer "F.Cu") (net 7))
 (segment (start 145.0767 90.1435) (end 145.0768 90.1435) (width 0.2) (layer "F.Cu") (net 7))
 (segment (start 146.185 96.655) (end 150.955 96.655) (width 0.2) (layer "F.Cu") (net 7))
 (segment (start 145.1905 73.5037) (end 146.1542 72.54) (width 0.2) (layer "F.Cu") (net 7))
 (segment (start 144.1138 65.8837) (end 145.0897 65.8837) (width 0.2) (layer "F.Cu") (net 7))
 (segment (start 145.1905 73.5037) (end 145.3953 73.5037) (width 0.2) (layer "F.Cu") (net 7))
 (segment (start 145.7058 96.6936) (end 145.7444 96.655) (width 0.2) (layer "F.Cu") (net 7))
 (segment (start 144 90.8837) (end 145.0767 90.8837) (width 0.2) (layer "F.Cu") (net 7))
 (segment (start 145.3167 65.7575) (end 145.1905 65.8837) (width 0.2) (layer "F.Cu") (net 7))
 (via (at 145.3953 70.5412) (size 0.6) (drill 0.3) (layers "F.Cu" "B.Cu") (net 7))
 (via (at 145.3953 73.5037) (size 0.6) (drill 0.3) (layers "F.Cu" "B.Cu") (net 7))
 (via (at 145.0768 90.1435) (size 0.6) (drill 0.3) (layers "F.Cu" "B.Cu") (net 7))
 (via (at 146.185 96.655) (size 0.6) (drill 0.3) (layers "F.Cu" "B.Cu") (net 7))
 (segment (start 145.3953 73.5037) (end 145.3953 70.5412) (width 0.2) (layer "B.Cu") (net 7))
 (segment (start 145.0768 95.5468) (end 145.0768 90.1435) (width 0.2) (layer "B.Cu") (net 7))
 (segment (start 145.0768 90.1435) (end 145.0768 73.8222) (width 0.2) (layer "B.Cu") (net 7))
 (segment (start 146.185 96.655) (end 145.0768 95.5468) (width 0.2) (layer "B.Cu") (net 7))
 (segment (start 145.0768 73.8222) (end 145.3953 73.5037) (width 0.2) (layer "B.Cu") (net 7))
 (segment (start 175.8625 79.58) (end 168.5 79.58) (width 0.2) (layer "F.Cu") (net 1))
 (segment (start 177.5 77.9425) (end 175.8625 79.58) (width 0.2) (layer "F.Cu") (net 1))
 (segment (start 175.96 75) (end 175.96 76.6225) (width 0.2) (layer "B.Cu") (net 1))
 (segment (start 176.18 76.6225) (end 177.5 77.9425) (width 0.2) (layer "B.Cu") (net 1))
 (segment (start 175.96 76.6225) (end 176.18 76.6225) (width 0.2) (layer "B.Cu") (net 1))
 (segment (start 149.92 79.3287) (end 151.2885 80.6972) (width 0.2) (layer "F.Cu") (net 13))
 (segment (start 151.2885 80.6972) (end 174.9979 80.6972) (width 0.2) (layer "F.Cu") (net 13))
 (via (at 174.9979 80.6972) (size 0.6) (drill 0.3) (layers "F.Cu" "B.Cu") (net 13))
 (segment (start 175.96 69.0025) (end 174.9979 69.9646) (width 0.2) (layer "B.Cu") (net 13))
 (segment (start 174.9979 69.9646) (end 174.9979 80.6972) (width 0.2) (layer "B.Cu") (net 13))
 (segment (start 146.8888 82.3599) (end 146.8888 86.3287) (width 0.2) (layer "B.Cu") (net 13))
 (segment (start 149.92 79.3287) (end 146.8888 82.3599) (width 0.2) (layer "B.Cu") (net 13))
 (segment (start 175.96 67.38) (end 175.96 69.0025) (width 0.2) (layer "B.Cu") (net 13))
 (segment (start 140.4971 67.1537) (end 139.7405 67.1537) (width 0.2) (layer "F.Cu") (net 17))
 (segment (start 139.7405 67.1537) (end 138.6638 67.1537) (width 0.2) (layer "F.Cu") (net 17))
 (segment (start 144.1138 69.6937) (end 143.0371 69.6937) (width 0.2) (layer "F.Cu") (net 17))
 (segment (start 143.0371 69.6937) (end 140.4971 67.1537) (width 0.2) (layer "F.Cu") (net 17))
 (segment (start 138.6638 65.8837) (end 139.7405 65.8837) (width 0.2) (layer "F.Cu") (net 17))
 (segment (start 139.7405 67.1537) (end 139.7405 65.8837) (width 0.2) (layer "F.Cu") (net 17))
 (segment (start 141.1755 72.8604) (end 143.0371 74.722) (width 0.2) (layer "F.Cu") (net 20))
 (segment (start 144.1138 74.7737) (end 143.0371 74.7737) (width 0.2) (layer "F.Cu") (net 20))
 (segment (start 144.1138 67.1537) (end 143.138 67.1537) (width 0.2) (layer "F.Cu") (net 20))
 (segment (start 142.4104 72.8604) (end 143.0371 72.2337) (width 0.2) (layer "F.Cu") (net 20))
 (segment (start 130.6101 68.0911) (end 130.6101 69.0283) (width 0.2) (layer "F.Cu") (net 20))
 (segment (start 133.4442 65.257) (end 130.6101 68.0911) (width 0.2) (layer "F.Cu") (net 20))
 (segment (start 143.6259 68.4237) (end 144.1138 68.4237) (width 0.2) (layer "F.Cu") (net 20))
 (segment (start 143.0386 67.1537) (end 143.0371 67.1537) (width 0.2) (layer "F.Cu") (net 20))
 (segment (start 144.1138 72.2337) (end 143.0371 72.2337) (width 0.2) (layer "F.Cu") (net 20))
 (segment (start 143.6259 68.4237) (end 143.138 68.4237) (width 0.2) (layer "F.Cu") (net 20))
 (segment (start 130.6101 69.0283) (end 134.4422 72.8604) (width 0.2) (layer "F.Cu") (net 20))
 (segment (start 143.138 68.4237) (end 143.0386 68.4237) (width 0.2) (layer "F.Cu") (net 20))
 (segment (start 143.0386 68.4237) (end 143.0371 68.4237) (width 0.2) (layer "F.Cu") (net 20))
 (segment (start 141.1755 72.8604) (end 142.4104 72.8604) (width 0.2) (layer "F.Cu") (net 20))
 (segment (start 134.4422 72.8604) (end 141.1755 72.8604) (width 0.2) (layer "F.Cu") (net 20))
 (segment (start 143.0371 74.722) (end 143.0371 74.7737) (width 0.2) (layer "F.Cu") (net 20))
 (segment (start 143.0386 67.1537) (end 141.1419 65.257) (width 0.2) (layer "F.Cu") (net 20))
 (segment (start 143.0371 67.1537) (end 143.0371 68.4237) (width 0.2) (layer "F.Cu") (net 20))
 (segment (start 141.1419 65.257) (end 133.4442 65.257) (width 0.2) (layer "F.Cu") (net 20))
 (segment (start 143.138 67.1537) (end 143.0386 67.1537) (width 0.2) (layer "F.Cu") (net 20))
 (segment (start 137.5871 72.2337) (end 137.5871 71.7199) (width 0.2) (layer "F.Cu") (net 6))
 (segment (start 150.1346 71.5904) (end 150.455 71.27) (width 0.2) (layer "F.Cu") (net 6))
 (segment (start 137.5871 71.7199) (end 137.7166 71.5904) (width 0.2) (layer "F.Cu") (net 6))
 (segment (start 138.1255 72.2337) (end 138.6638 72.2337) (width 0.2) (layer "F.Cu") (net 6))
 (segment (start 138.1255 72.2337) (end 137.5871 72.2337) (width 0.2) (layer "F.Cu") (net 6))
 (segment (start 138.6638 70.9637) (end 139.5742 70.9637) (width 0.2) (layer "F.Cu") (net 6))
 (segment (start 137.7166 71.5904) (end 139.5742 71.5904) (width 0.2) (layer "F.Cu") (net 6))
 (segment (start 139.5742 71.5904) (end 150.1346 71.5904) (width 0.2) (layer "F.Cu") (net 6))
 (segment (start 139.5742 70.9637) (end 139.5742 71.5904) (width 0.2) (layer "F.Cu") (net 6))
 (segment (start 147.0488 79.3287) (end 144.2955 79.3287) (width 0.2) (layer "F.Cu") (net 19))
 (segment (start 144.2955 79.3287) (end 139.7405 74.7737) (width 0.2) (layer "F.Cu") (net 19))
 (segment (start 139.2022 74.7737) (end 139.7405 74.7737) (width 0.2) (layer "F.Cu") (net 19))
 (segment (start 139.2022 74.7737) (end 139.7405 74.2354) (width 0.2) (layer "F.Cu") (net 19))
 (segment (start 138.6638 74.7737) (end 139.2022 74.7737) (width 0.2) (layer "F.Cu") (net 19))
 (segment (start 139.7405 74.2354) (end 139.7405 73.5037) (width 0.2) (layer "F.Cu") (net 19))
 (segment (start 138.6638 73.5037) (end 139.7405 73.5037) (width 0.2) (layer "F.Cu") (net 19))
 (segment (start 143.5625 93.4237) (end 143.0242 93.4237) (width 0.2) (layer "F.Cu") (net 23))
 (segment (start 144 93.4237) (end 146.8075 93.4237) (width 0.2) (layer "F.Cu") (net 23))
 (segment (start 144.4375 99.7737) (end 145.0767 99.7737) (width 0.2) (layer "F.Cu") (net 23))
 (segment (start 142.9233 92.1537) (end 142.9233 93.4237) (width 0.2) (layer "F.Cu") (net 23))
 (segment (start 145.2191 99.9161) (end 146.8075 99.9161) (width 0.2) (layer "F.Cu") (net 23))
 (segment (start 145.0767 99.7737) (end 145.2191 99.9161) (width 0.2) (layer "F.Cu") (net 23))
 (segment (start 144 92.1537) (end 142.9233 92.1537) (width 0.2) (layer "F.Cu") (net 23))
 (segment (start 142.9248 93.4237) (end 142.9233 93.4237) (width 0.2) (layer "F.Cu") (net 23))
 (segment (start 143.5625 93.4237) (end 144 93.4237) (width 0.2) (layer "F.Cu") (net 23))
 (segment (start 144.4375 99.7737) (end 144 99.7737) (width 0.2) (layer "F.Cu") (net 23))
 (segment (start 143.0242 93.4237) (end 142.9248 93.4237) (width 0.2) (layer "F.Cu") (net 23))
 (via (at 146.8075 99.9161) (size 0.6) (drill 0.3) (layers "F.Cu" "B.Cu") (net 23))
 (via (at 146.8075 93.4237) (size 0.6) (drill 0.3) (layers "F.Cu" "B.Cu") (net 23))
 (segment (start 146.8075 99.9161) (end 146.8075 93.4237) (width 0.2) (layer "B.Cu") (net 23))
 (segment (start 144 94.6937) (end 142.9233 94.6937) (width 0.2) (layer "F.Cu") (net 21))
 (segment (start 140.3833 92.1537) (end 139.6267 92.1537) (width 0.2) (layer "F.Cu") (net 21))
 (segment (start 142.9233 94.6937) (end 140.3833 92.1537) (width 0.2) (layer "F.Cu") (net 21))
 (segment (start 139.6267 92.1537) (end 138.55 92.1537) (width 0.2) (layer "F.Cu") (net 21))
 (segment (start 138.55 90.8837) (end 139.6267 90.8837) (width 0.2) (layer "F.Cu") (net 21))
 (segment (start 139.6267 90.8837) (end 139.6267 92.1537) (width 0.2) (layer "F.Cu") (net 21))
 (segment (start 137.4733 99.6573) (end 132.1319 99.6573) (width 0.2) (layer "F.Cu") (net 11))
 (segment (start 131.5612 89.3475) (end 133 87.9087) (width 0.2) (layer "F.Cu") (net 11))
 (segment (start 131.5612 99.0866) (end 131.5612 89.3475) (width 0.2) (layer "F.Cu") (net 11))
 (segment (start 137.4733 99.7737) (end 137.4733 99.6573) (width 0.2) (layer "F.Cu") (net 11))
 (segment (start 137.4733 99.6573) (end 137.4733 98.5037) (width 0.2) (layer "F.Cu") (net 11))
 (segment (start 138.55 99.7737) (end 137.4733 99.7737) (width 0.2) (layer "F.Cu") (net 11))
 (segment (start 132.1319 99.6573) (end 131.5612 99.0866) (width 0.2) (layer "F.Cu") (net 11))
 (segment (start 138.55 98.5037) (end 137.4733 98.5037) (width 0.2) (layer "F.Cu") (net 11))
 (segment (start 138.0117 95.9637) (end 137.4733 95.9637) (width 0.2) (layer "F.Cu") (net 22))
 (segment (start 150.907 95.337) (end 150.955 95.385) (width 0.2) (layer "F.Cu") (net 22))
 (segment (start 139.6267 95.9637) (end 140.2534 95.337) (width 0.2) (layer "F.Cu") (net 22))
 (segment (start 140.2534 95.337) (end 150.907 95.337) (width 0.2) (layer "F.Cu") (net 22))
 (segment (start 138.0117 95.9637) (end 138.55 95.9637) (width 0.2) (layer "F.Cu") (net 22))
 (segment (start 138.55 97.2337) (end 137.4733 97.2337) (width 0.2) (layer "F.Cu") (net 22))
 (segment (start 137.4733 97.2337) (end 137.4733 95.9637) (width 0.2) (layer "F.Cu") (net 22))
 (segment (start 138.55 95.9637) (end 139.6267 95.9637) (width 0.2) (layer "F.Cu") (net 22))
 (segment (start 161.433 79.58) (end 161.1817 79.3287) (width 0.2) (layer "F.Cu") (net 3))
 (segment (start 155.8136 71.27) (end 160.08 75.5364) (width 0.2) (layer "F.Cu") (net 3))
 (segment (start 155.405 71.27) (end 155.8136 71.27) (width 0.2) (layer "F.Cu") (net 3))
 (segment (start 160.08 79.3287) (end 161.1817 79.3287) (width 0.2) (layer "F.Cu") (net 3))
 (segment (start 160.08 75.5364) (end 160.08 79.3287) (width 0.2) (layer "F.Cu") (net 3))
 (segment (start 163.5 79.58) (end 161.433 79.58) (width 0.2) (layer "F.Cu") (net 3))
 (segment (start 161.1053 68.127) (end 162.3983 69.42) (width 0.2) (layer "F.Cu") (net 4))
 (segment (start 150.0466 70) (end 149.1465 69.0999) (width 0.2) (layer "F.Cu") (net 4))
 (segment (start 163.5 69.42) (end 162.3983 69.42) (width 0.2) (layer "F.Cu") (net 4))
 (segment (start 150.455 70) (end 150.0466 70) (width 0.2) (layer "F.Cu") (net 4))
 (segment (start 149.1465 69.0999) (end 149.1465 68.3931) (width 0.2) (layer "F.Cu") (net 4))
 (segment (start 149.1465 68.3931) (end 149.4126 68.127) (width 0.2) (layer "F.Cu") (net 4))
 (segment (start 149.4126 68.127) (end 161.1053 68.127) (width 0.2) (layer "F.Cu") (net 4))
 (segment (start 155.905 95.385) (end 156.4113 95.385) (width 0.2) (layer "F.Cu") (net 5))
 (segment (start 156.4113 95.385) (end 160 91.7963) (width 0.2) (layer "F.Cu") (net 5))
 (segment (start 160 91.7963) (end 160 86.3287) (width 0.2) (layer "F.Cu") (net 5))
 (segment (start 163.5 85.92) (end 160.4087 85.92) (width 0.2) (layer "F.Cu") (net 5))
 (segment (start 160.4087 85.92) (end 160 86.3287) (width 0.2) (layer "F.Cu") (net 5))
 (segment (start 150.955 94.115) (end 149.4741 94.115) (width 0.2) (layer "F.Cu") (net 26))
 (via (at 149.4741 94.115) (size 0.6) (drill 0.3) (layers "F.Cu" "B.Cu") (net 26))
 (segment (start 149.84 86.3287) (end 149.84 93.7491) (width 0.2) (layer "B.Cu") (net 26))
 (segment (start 149.84 93.7491) (end 149.4741 94.115) (width 0.2) (layer "B.Cu") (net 26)))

